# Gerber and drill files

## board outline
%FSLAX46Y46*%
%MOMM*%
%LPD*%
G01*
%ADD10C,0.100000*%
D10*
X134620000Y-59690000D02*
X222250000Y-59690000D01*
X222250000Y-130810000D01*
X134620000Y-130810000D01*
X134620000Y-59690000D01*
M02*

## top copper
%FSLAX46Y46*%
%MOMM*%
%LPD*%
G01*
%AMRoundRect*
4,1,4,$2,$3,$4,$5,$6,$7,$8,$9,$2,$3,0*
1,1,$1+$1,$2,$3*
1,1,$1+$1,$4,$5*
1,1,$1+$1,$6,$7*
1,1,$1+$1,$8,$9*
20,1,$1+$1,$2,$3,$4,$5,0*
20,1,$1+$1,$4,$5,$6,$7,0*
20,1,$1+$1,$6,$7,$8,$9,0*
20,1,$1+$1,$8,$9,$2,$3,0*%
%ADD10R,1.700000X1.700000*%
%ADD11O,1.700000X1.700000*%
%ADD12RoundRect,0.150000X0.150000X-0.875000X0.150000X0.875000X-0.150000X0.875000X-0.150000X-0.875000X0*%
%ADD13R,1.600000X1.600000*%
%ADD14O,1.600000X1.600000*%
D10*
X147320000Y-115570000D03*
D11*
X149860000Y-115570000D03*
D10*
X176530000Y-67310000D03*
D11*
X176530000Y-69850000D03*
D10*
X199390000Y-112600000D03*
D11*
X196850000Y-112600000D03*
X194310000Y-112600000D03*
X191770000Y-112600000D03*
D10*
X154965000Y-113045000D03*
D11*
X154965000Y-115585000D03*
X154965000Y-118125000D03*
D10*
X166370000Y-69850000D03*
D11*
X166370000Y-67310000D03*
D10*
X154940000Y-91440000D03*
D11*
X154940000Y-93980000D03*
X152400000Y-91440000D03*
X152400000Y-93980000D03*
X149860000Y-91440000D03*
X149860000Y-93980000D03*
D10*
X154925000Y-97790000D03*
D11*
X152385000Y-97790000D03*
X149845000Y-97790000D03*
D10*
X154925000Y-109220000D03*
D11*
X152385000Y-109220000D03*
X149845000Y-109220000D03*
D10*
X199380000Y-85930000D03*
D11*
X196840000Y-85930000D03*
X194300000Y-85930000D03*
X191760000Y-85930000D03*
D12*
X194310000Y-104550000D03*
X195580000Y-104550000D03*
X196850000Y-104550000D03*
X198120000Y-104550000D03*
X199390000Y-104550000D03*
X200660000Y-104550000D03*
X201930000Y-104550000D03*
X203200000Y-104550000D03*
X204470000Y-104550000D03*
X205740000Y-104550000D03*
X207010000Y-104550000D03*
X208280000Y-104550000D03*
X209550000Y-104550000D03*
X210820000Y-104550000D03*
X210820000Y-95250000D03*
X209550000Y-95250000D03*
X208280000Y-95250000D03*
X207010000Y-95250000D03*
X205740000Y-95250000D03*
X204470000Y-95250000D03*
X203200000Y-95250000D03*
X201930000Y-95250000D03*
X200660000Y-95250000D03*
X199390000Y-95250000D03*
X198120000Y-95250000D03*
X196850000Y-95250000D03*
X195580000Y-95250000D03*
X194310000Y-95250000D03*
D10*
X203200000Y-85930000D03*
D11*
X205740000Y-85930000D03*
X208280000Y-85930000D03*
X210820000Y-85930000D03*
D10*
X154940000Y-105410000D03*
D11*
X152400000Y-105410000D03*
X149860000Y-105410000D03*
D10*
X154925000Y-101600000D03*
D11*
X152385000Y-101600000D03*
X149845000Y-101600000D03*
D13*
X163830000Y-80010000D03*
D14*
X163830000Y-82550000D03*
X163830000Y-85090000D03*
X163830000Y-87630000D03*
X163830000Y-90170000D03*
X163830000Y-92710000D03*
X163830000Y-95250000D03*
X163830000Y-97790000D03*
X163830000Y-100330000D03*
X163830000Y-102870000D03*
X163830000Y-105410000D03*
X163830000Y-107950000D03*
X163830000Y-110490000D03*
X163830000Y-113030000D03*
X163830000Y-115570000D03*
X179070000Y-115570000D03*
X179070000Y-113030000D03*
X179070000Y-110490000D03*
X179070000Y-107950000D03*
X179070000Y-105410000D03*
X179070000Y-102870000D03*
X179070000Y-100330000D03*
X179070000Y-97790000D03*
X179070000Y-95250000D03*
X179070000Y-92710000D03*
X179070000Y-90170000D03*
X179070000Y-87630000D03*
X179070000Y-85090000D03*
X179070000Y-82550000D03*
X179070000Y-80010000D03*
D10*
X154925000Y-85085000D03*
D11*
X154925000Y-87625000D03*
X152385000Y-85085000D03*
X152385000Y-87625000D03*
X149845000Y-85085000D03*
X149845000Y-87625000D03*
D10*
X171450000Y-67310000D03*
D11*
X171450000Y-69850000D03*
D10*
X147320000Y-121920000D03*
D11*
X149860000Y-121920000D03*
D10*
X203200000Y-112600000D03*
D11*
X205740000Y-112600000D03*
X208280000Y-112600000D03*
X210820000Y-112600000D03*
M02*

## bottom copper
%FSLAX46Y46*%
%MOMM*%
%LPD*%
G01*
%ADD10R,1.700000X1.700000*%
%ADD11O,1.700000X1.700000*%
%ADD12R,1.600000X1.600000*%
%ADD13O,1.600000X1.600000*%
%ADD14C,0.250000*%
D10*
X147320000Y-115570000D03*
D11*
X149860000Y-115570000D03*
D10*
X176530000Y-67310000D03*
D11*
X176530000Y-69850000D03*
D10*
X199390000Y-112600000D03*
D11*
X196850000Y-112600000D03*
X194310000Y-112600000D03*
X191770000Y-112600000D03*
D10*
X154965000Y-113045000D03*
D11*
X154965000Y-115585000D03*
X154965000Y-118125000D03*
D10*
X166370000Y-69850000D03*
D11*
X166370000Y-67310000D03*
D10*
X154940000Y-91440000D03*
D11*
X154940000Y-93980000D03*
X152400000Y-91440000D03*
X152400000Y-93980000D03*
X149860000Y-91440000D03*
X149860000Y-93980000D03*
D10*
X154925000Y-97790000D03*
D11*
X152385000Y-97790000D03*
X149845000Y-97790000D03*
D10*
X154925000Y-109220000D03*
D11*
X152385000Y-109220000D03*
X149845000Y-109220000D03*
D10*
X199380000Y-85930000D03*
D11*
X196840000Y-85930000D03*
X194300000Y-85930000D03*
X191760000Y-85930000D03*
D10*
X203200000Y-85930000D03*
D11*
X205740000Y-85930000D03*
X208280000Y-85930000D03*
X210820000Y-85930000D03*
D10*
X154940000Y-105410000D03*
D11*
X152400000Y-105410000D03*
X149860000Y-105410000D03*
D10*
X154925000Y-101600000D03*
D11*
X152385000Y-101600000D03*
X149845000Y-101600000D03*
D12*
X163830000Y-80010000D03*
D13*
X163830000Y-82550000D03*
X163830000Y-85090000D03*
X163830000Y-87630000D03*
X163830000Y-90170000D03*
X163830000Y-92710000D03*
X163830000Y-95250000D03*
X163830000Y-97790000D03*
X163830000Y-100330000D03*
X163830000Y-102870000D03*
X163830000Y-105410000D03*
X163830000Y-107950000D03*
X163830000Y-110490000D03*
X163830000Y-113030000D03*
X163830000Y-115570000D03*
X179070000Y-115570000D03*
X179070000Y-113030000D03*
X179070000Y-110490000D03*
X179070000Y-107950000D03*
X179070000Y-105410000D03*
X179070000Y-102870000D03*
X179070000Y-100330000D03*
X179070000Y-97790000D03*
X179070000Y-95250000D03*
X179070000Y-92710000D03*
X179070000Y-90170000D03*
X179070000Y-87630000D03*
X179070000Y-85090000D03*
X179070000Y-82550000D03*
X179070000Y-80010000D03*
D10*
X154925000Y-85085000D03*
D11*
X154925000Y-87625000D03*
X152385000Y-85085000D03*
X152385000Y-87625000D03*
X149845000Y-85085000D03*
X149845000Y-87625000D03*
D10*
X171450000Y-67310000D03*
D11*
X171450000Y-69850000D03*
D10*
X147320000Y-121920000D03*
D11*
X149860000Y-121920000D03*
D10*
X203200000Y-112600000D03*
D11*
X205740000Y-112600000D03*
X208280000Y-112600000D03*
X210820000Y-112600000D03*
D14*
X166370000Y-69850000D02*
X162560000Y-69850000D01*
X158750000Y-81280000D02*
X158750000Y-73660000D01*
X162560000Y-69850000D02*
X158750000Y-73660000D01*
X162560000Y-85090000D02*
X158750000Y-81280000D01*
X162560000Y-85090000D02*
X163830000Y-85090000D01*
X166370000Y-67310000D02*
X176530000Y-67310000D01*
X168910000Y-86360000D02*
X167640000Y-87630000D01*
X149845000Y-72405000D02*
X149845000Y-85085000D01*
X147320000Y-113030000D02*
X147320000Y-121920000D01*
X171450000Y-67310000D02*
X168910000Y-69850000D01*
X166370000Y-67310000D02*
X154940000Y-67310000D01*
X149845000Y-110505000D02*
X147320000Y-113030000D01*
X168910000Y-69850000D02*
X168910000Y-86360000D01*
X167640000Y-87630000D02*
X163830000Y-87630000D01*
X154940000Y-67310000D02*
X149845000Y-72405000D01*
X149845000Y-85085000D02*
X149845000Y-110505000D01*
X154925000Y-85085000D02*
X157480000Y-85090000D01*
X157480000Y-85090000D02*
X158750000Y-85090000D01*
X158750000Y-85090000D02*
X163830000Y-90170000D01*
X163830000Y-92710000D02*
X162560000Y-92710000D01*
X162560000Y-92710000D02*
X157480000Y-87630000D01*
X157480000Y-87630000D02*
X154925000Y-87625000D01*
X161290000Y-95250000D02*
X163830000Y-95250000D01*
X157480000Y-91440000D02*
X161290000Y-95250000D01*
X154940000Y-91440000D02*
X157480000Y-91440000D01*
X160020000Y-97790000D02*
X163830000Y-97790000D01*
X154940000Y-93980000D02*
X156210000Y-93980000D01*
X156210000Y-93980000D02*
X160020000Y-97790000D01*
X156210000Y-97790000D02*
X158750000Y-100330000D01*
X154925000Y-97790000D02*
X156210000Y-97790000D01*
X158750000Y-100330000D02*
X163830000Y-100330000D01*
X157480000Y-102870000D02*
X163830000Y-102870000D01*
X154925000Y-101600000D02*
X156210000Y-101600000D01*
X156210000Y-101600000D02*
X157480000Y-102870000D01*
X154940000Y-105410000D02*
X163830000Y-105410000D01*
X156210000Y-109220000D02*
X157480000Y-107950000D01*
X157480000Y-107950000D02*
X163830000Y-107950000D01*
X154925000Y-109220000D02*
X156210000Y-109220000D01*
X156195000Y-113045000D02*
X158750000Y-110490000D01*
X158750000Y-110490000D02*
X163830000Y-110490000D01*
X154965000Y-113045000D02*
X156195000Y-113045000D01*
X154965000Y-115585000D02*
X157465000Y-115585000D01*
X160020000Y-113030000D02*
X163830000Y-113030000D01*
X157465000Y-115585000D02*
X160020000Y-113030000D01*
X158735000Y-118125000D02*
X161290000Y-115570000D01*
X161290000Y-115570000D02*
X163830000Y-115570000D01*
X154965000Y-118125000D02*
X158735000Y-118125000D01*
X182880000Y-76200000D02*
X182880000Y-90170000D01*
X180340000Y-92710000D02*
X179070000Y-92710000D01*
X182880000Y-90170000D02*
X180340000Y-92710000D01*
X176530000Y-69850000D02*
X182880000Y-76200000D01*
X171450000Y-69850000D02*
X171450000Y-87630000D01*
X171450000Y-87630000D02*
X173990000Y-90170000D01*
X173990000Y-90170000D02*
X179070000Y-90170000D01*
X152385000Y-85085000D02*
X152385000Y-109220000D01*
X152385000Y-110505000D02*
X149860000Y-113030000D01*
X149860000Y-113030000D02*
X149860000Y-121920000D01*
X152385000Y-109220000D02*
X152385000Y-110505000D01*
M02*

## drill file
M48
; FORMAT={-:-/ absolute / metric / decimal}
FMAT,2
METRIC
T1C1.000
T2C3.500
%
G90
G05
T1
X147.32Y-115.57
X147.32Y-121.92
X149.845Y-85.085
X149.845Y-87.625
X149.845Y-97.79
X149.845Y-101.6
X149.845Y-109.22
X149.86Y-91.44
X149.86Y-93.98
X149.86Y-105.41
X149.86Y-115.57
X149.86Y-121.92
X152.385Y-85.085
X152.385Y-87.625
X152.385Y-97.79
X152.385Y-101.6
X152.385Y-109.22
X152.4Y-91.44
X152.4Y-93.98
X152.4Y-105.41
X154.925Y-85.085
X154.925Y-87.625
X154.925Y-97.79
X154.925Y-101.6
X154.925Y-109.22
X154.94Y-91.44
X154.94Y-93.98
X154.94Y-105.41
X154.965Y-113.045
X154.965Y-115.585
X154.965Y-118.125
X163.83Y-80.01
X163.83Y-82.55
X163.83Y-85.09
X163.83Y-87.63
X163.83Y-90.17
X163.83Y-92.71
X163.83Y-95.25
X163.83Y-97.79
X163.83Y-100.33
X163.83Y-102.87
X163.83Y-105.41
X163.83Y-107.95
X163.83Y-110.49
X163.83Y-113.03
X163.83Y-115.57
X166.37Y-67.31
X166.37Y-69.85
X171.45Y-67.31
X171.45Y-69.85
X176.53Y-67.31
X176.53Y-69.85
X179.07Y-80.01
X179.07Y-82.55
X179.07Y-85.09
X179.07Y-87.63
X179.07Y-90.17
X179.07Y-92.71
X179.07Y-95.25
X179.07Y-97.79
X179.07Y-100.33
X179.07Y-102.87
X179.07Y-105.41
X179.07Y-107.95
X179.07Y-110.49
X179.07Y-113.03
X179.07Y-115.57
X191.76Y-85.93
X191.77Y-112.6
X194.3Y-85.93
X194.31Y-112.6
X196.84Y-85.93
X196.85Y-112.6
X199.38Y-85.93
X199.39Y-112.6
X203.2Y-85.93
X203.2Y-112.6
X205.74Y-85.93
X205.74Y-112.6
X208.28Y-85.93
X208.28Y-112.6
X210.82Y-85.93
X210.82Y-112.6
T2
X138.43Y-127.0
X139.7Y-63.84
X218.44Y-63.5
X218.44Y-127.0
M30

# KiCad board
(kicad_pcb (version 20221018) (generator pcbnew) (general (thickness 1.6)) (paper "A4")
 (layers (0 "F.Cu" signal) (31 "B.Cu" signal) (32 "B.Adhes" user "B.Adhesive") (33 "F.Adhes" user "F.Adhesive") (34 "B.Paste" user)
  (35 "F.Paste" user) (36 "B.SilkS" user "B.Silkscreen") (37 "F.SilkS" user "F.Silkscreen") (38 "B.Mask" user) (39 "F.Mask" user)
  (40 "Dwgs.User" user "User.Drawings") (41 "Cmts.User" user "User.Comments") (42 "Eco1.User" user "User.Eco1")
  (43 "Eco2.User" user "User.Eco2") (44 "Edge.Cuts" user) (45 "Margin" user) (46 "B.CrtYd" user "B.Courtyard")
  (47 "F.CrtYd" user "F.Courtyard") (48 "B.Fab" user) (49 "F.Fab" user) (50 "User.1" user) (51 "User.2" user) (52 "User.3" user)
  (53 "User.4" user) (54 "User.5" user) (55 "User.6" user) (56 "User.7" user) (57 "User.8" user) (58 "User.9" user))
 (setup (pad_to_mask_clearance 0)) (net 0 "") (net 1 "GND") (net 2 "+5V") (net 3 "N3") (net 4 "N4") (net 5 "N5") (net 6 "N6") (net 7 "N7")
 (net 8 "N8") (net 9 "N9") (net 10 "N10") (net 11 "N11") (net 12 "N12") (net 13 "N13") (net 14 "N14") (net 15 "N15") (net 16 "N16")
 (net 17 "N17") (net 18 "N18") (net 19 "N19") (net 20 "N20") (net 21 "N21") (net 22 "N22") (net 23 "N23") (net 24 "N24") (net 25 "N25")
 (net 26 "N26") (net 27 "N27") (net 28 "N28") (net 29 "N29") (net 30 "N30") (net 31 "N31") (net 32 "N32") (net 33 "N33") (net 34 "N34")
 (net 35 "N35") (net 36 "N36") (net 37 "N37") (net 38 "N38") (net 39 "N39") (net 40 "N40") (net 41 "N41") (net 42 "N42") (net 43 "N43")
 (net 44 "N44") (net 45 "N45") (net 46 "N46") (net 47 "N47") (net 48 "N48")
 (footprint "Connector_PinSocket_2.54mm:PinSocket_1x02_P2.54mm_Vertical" (layer "F.Cu") (at 147.32 115.57 90)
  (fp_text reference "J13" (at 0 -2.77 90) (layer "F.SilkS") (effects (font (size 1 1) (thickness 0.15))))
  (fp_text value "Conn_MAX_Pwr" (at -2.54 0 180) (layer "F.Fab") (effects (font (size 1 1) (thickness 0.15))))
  (pad "1" thru_hole rect (at 0 0 90) (size 1.7 1.7) (drill 1) (layers "*.Cu" "*.Mask") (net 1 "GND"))
  (pad "2" thru_hole oval (at 0 2.54 90) (size 1.7 1.7) (drill 1) (layers "*.Cu" "*.Mask") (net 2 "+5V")))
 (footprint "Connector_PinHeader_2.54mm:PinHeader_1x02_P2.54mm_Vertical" (layer "F.Cu") (at 176.53 67.31)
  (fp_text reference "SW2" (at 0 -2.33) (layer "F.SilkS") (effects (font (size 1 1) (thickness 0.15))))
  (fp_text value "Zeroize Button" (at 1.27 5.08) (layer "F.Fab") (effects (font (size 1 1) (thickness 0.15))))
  (pad "1" thru_hole rect (at 0 0) (size 1.7 1.7) (drill 1) (layers "*.Cu" "*.Mask") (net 1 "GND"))
  (pad "2" thru_hole oval (at 0 2.54) (size 1.7 1.7) (drill 1) (layers "*.Cu" "*.Mask") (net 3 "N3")))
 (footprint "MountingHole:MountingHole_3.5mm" (layer "F.Cu") (at 139.7 63.84)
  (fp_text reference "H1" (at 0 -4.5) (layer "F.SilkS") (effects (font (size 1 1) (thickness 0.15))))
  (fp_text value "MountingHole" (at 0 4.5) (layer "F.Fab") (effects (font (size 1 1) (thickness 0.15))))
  (pad "" np_thru_hole circle (at 0 0) (size 3.5 3.5) (drill 3.5) (layers "*.Cu" "*.Mask")))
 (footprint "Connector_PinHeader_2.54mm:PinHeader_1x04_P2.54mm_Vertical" (layer "F.Cu") (at 199.39 112.6 -90)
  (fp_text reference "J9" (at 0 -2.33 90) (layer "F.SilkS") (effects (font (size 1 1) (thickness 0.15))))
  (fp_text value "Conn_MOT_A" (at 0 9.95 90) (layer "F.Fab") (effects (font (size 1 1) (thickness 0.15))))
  (pad "1" thru_hole rect (at 0 0 270) (size 1.7 1.7) (drill 1) (layers "*.Cu" "*.Mask") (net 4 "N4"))
  (pad "2" thru_hole oval (at 0 2.54 270) (size 1.7 1.7) (drill 1) (layers "*.Cu" "*.Mask") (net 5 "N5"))
  (pad "3" thru_hole oval (at 0 5.08 270) (size 1.7 1.7) (drill 1) (layers "*.Cu" "*.Mask") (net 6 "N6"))
  (pad "4" thru_hole oval (at 0 7.62 270) (size 1.7 1.7) (drill 1) (layers "*.Cu" "*.Mask") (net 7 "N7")))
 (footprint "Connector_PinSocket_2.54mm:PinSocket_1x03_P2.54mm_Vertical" (layer "F.Cu") (at 154.965 113.045)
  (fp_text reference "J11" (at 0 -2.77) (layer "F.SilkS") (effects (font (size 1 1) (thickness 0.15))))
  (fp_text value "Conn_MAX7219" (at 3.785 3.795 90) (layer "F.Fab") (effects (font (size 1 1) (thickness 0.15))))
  (pad "1" thru_hole rect (at 0 0) (size 1.7 1.7) (drill 1) (layers "*.Cu" "*.Mask") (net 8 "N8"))
  (pad "2" thru_hole oval (at 0 2.54) (size 1.7 1.7) (drill 1) (layers "*.Cu" "*.Mask") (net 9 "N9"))
  (pad "3" thru_hole oval (at 0 5.08) (size 1.7 1.7) (drill 1) (layers "*.Cu" "*.Mask") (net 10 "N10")))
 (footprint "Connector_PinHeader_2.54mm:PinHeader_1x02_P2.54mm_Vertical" (layer "F.Cu") (at 166.37 69.85 180)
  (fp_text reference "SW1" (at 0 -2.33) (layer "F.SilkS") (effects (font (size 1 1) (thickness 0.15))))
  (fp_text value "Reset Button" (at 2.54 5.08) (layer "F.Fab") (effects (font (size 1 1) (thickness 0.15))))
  (pad "1" thru_hole rect (at 0 0 180) (size 1.7 1.7) (drill 1) (layers "*.Cu" "*.Mask") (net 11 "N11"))
  (pad "2" thru_hole oval (at 0 2.54 180) (size 1.7 1.7) (drill 1) (layers "*.Cu" "*.Mask") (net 1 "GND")))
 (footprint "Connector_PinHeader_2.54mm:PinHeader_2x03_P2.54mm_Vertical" (layer "F.Cu") (at 154.94 91.44 -90)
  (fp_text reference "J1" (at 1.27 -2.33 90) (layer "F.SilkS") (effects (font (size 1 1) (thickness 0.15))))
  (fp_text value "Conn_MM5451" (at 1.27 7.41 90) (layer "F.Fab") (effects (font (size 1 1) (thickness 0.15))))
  (pad "1" thru_hole rect (at 0 0 270) (size 1.7 1.7) (drill 1) (layers "*.Cu" "*.Mask") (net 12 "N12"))
  (pad "2" thru_hole oval (at 2.54 0 270) (size 1.7 1.7) (drill 1) (layers "*.Cu" "*.Mask") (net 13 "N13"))
  (pad "3" thru_hole oval (at 0 2.54 270) (size 1.7 1.7) (drill 1) (layers "*.Cu" "*.Mask") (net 2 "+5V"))
  (pad "4" thru_hole oval (at 2.54 2.54 270) (size 1.7 1.7) (drill 1) (layers "*.Cu" "*.Mask") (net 2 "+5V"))
  (pad "5" thru_hole oval (at 0 5.08 270) (size 1.7 1.7) (drill 1) (layers "*.Cu" "*.Mask") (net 1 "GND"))
  (pad "6" thru_hole oval (at 2.54 5.08 270) (size 1.7 1.7) (drill 1) (layers "*.Cu" "*.Mask") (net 1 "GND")))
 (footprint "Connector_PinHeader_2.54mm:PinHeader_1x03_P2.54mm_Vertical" (layer "F.Cu") (at 154.925 97.79 -90)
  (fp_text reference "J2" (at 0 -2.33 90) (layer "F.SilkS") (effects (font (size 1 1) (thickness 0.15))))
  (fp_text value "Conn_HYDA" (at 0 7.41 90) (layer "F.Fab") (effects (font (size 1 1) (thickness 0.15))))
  (pad "1" thru_hole rect (at 0 0 270) (size 1.7 1.7) (drill 1) (layers "*.Cu" "*.Mask") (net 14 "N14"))
  (pad "2" thru_hole oval (at 0 2.54 270) (size 1.7 1.7) (drill 1) (layers "*.Cu" "*.Mask") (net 2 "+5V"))
  (pad "3" thru_hole oval (at 0 5.08 270) (size 1.7 1.7) (drill 1) (layers "*.Cu" "*.Mask") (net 1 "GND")))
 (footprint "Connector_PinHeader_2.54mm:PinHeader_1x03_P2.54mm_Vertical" (layer "F.Cu") (at 154.925 109.22 -90)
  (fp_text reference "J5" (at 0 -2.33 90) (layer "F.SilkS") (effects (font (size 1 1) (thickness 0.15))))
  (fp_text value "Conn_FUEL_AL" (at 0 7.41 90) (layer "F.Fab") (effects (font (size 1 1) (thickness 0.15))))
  (pad "1" thru_hole rect (at 0 0 270) (size 1.7 1.7) (drill 1) (layers "*.Cu" "*.Mask") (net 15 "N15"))
  (pad "2" thru_hole oval (at 0 2.54 270) (size 1.7 1.7) (drill 1) (layers "*.Cu" "*.Mask") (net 2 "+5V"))
  (pad "3" thru_hole oval (at 0 5.08 270) (size 1.7 1.7) (drill 1) (layers "*.Cu" "*.Mask") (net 1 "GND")))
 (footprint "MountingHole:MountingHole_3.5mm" (layer "F.Cu") (at 218.44 127)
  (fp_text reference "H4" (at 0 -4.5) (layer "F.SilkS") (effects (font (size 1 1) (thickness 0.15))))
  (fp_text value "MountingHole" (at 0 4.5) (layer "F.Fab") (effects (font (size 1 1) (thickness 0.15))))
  (pad "" np_thru_hole circle (at 0 0) (size 3.5 3.5) (drill 3.5) (layers "*.Cu" "*.Mask")))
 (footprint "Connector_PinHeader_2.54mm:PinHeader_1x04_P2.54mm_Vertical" (layer "F.Cu") (at 199.38 85.93 -90)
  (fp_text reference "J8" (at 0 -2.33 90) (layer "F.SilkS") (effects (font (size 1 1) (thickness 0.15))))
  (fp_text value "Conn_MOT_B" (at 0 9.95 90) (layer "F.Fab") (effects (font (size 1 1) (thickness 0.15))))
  (pad "1" thru_hole rect (at 0 0 270) (size 1.7 1.7) (drill 1) (layers "*.Cu" "*.Mask") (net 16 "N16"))
  (pad "2" thru_hole oval (at 0 2.54 270) (size 1.7 1.7) (drill 1) (layers "*.Cu" "*.Mask") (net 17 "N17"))
  (pad "3" thru_hole oval (at 0 5.08 270) (size 1.7 1.7) (drill 1) (layers "*.Cu" "*.Mask") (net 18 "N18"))
  (pad "4" thru_hole oval (at 0 7.62 270) (size 1.7 1.7) (drill 1) (layers "*.Cu" "*.Mask") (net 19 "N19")))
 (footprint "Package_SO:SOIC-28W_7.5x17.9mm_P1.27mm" (layer "F.Cu") (at 202.565 99.9 90)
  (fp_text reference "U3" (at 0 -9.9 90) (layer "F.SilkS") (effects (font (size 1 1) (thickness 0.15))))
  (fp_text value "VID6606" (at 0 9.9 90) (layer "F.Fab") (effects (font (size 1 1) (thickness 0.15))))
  (pad "1" smd roundrect (at -4.65 -8.255 90) (size 2.05 0.6) (layers "F.Cu" "F.Paste" "F.Mask") (roundrect_rratio 0.25) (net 1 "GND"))
  (pad "2" smd roundrect (at -4.65 -6.985 90) (size 2.05 0.6) (layers "F.Cu" "F.Paste" "F.Mask") (roundrect_rratio 0.25) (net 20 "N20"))
  (pad "3" smd roundrect (at -4.65 -5.715 90) (size 2.05 0.6) (layers "F.Cu" "F.Paste" "F.Mask") (roundrect_rratio 0.25) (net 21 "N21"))
  (pad "4" smd roundrect (at -4.65 -4.445 90) (size 2.05 0.6) (layers "F.Cu" "F.Paste" "F.Mask") (roundrect_rratio 0.25) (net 7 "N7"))
  (pad "5" smd roundrect (at -4.65 -3.175 90) (size 2.05 0.6) (layers "F.Cu" "F.Paste" "F.Mask") (roundrect_rratio 0.25) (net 6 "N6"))
  (pad "6" smd roundrect (at -4.65 -1.905 90) (size 2.05 0.6) (layers "F.Cu" "F.Paste" "F.Mask") (roundrect_rratio 0.25) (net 5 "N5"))
  (pad "7" smd roundrect (at -4.65 -0.635 90) (size 2.05 0.6) (layers "F.Cu" "F.Paste" "F.Mask") (roundrect_rratio 0.25) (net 4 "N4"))
  (pad "8" smd roundrect (at -4.65 0.635 90) (size 2.05 0.6) (layers "F.Cu" "F.Paste" "F.Mask") (roundrect_rratio 0.25) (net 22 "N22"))
  (pad "9" smd roundrect (at -4.65 1.905 90) (size 2.05 0.6) (layers "F.Cu" "F.Paste" "F.Mask") (roundrect_rratio 0.25) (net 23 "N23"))
  (pad "10" smd roundrect (at -4.65 3.175 90) (size 2.05 0.6) (layers "F.Cu" "F.Paste" "F.Mask") (roundrect_rratio 0.25) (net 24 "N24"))
  (pad "11" smd roundrect (at -4.65 4.445 90) (size 2.05 0.6) (layers "F.Cu" "F.Paste" "F.Mask") (roundrect_rratio 0.25) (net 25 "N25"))
  (pad "12" smd roundrect (at -4.65 5.715 90) (size 2.05 0.6) (layers "F.Cu" "F.Paste" "F.Mask") (roundrect_rratio 0.25) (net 2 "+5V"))
  (pad "13" smd roundrect (at -4.65 6.985 90) (size 2.05 0.6) (layers "F.Cu" "F.Paste" "F.Mask") (roundrect_rratio 0.25) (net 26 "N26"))
  (pad "14" smd roundrect (at -4.65 8.255 90) (size 2.05 0.6) (layers "F.Cu" "F.Paste" "F.Mask") (roundrect_rratio 0.25) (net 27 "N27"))
  (pad "15" smd roundrect (at 4.65 8.255 90) (size 2.05 0.6) (layers "F.Cu" "F.Paste" "F.Mask") (roundrect_rratio 0.25) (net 1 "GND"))
  (pad "16" smd roundrect (at 4.65 6.985 90) (size 2.05 0.6) (layers "F.Cu" "F.Paste" "F.Mask") (roundrect_rratio 0.25) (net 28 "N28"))
  (pad "17" smd roundrect (at 4.65 5.715 90) (size 2.05 0.6) (layers "F.Cu" "F.Paste" "F.Mask") (roundrect_rratio 0.25) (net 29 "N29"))
  (pad "18" smd roundrect (at 4.65 4.445 90) (size 2.05 0.6) (layers "F.Cu" "F.Paste" "F.Mask") (roundrect_rratio 0.25) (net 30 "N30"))
  (pad "19" smd roundrect (at 4.65 3.175 90) (size 2.05 0.6) (layers "F.Cu" "F.Paste" "F.Mask") (roundrect_rratio 0.25) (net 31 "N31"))
  (pad "20" smd roundrect (at 4.65 1.905 90) (size 2.05 0.6) (layers "F.Cu" "F.Paste" "F.Mask") (roundrect_rratio 0.25) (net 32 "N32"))
  (pad "21" smd roundrect (at 4.65 0.635 90) (size 2.05 0.6) (layers "F.Cu" "F.Paste" "F.Mask") (roundrect_rratio 0.25) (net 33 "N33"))
  (pad "22" smd roundrect (at 4.65 -0.635 90) (size 2.05 0.6) (layers "F.Cu" "F.Paste" "F.Mask") (roundrect_rratio 0.25) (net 16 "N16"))
  (pad "23" smd roundrect (at 4.65 -1.905 90) (size 2.05 0.6) (layers "F.Cu" "F.Paste" "F.Mask") (roundrect_rratio 0.25) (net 17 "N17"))
  (pad "24" smd roundrect (at 4.65 -3.175 90) (size 2.05 0.6) (layers "F.Cu" "F.Paste" "F.Mask") (roundrect_rratio 0.25) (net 18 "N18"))
  (pad "25" smd roundrect (at 4.65 -4.445 90) (size 2.05 0.6) (layers "F.Cu" "F.Paste" "F.Mask") (roundrect_rratio 0.25) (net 19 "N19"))
  (pad "26" smd roundrect (at 4.65 -5.715 90) (size 2.05 0.6) (layers "F.Cu" "F.Paste" "F.Mask") (roundrect_rratio 0.25) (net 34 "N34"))
  (pad "27" smd roundrect (at 4.65 -6.985 90) (size 2.05 0.6) (layers "F.Cu" "F.Paste" "F.Mask") (roundrect_rratio 0.25) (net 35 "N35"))
  (pad "28" smd roundrect (at 4.65 -8.255 90) (size 2.05 0.6) (layers "F.Cu" "F.Paste" "F.Mask") (roundrect_rratio 0.25) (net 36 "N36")))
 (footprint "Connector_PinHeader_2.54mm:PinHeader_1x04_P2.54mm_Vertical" (layer "F.Cu") (at 203.2 85.93 90)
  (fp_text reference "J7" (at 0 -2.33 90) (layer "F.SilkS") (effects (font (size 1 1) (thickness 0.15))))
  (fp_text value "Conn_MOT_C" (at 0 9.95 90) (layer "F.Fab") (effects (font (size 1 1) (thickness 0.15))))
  (pad "1" thru_hole rect (at 0 0 90) (size 1.7 1.7) (drill 1) (layers "*.Cu" "*.Mask") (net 33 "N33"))
  (pad "2" thru_hole oval (at 0 2.54 90) (size 1.7 1.7) (drill 1) (layers "*.Cu" "*.Mask") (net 32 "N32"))
  (pad "3" thru_hole oval (at 0 5.08 90) (size 1.7 1.7) (drill 1) (layers "*.Cu" "*.Mask") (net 31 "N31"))
  (pad "4" thru_hole oval (at 0 7.62 90) (size 1.7 1.7) (drill 1) (layers "*.Cu" "*.Mask") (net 30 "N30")))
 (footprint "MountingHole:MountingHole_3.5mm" (layer "F.Cu") (at 218.44 63.5)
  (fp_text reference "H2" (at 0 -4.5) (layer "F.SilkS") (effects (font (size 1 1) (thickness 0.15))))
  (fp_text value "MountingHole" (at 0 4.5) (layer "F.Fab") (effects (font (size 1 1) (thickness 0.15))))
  (pad "" np_thru_hole circle (at 0 0) (size 3.5 3.5) (drill 3.5) (layers "*.Cu" "*.Mask")))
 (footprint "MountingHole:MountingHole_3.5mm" (layer "F.Cu") (at 138.43 127)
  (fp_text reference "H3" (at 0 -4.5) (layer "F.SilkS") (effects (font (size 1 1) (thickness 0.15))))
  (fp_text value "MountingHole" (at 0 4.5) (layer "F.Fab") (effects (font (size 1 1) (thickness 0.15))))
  (pad "" np_thru_hole circle (at 0 0) (size 3.5 3.5) (drill 3.5) (layers "*.Cu" "*.Mask")))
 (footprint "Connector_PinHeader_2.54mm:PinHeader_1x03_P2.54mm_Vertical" (layer "F.Cu") (at 154.94 105.41 -90)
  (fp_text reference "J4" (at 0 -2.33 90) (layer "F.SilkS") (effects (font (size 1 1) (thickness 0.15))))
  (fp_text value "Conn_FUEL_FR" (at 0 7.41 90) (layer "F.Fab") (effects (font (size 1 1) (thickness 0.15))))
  (pad "1" thru_hole rect (at 0 0 270) (size 1.7 1.7) (drill 1) (layers "*.Cu" "*.Mask") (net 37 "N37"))
  (pad "2" thru_hole oval (at 0 2.54 270) (size 1.7 1.7) (drill 1) (layers "*.Cu" "*.Mask") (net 2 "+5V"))
  (pad "3" thru_hole oval (at 0 5.08 270) (size 1.7 1.7) (drill 1) (layers "*.Cu" "*.Mask") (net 1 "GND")))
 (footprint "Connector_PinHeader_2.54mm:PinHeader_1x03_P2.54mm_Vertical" (layer "F.Cu") (at 154.925 101.6 -90)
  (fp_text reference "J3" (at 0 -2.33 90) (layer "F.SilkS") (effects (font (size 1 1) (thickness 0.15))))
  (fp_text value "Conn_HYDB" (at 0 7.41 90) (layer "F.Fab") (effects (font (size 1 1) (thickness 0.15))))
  (pad "1" thru_hole rect (at 0 0 270) (size 1.7 1.7) (drill 1) (layers "*.Cu" "*.Mask") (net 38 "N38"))
  (pad "2" thru_hole oval (at 0 2.54 270) (size 1.7 1.7) (drill 1) (layers "*.Cu" "*.Mask") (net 2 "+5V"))
  (pad "3" thru_hole oval (at 0 5.08 270) (size 1.7 1.7) (drill 1) (layers "*.Cu" "*.Mask") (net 1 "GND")))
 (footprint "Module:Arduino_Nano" (layer "F.Cu") (at 163.83 80.01)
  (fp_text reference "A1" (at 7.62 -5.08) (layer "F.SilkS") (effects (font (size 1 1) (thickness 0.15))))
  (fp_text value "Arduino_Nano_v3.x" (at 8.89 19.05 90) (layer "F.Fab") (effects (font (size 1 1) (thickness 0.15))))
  (pad "1" thru_hole rect (at 0 0) (size 1.6 1.6) (drill 1) (layers "*.Cu" "*.Mask") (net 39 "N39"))
  (pad "2" thru_hole oval (at 0 2.54) (size 1.6 1.6) (drill 1) (layers "*.Cu" "*.Mask") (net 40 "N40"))
  (pad "3" thru_hole oval (at 0 5.08) (size 1.6 1.6) (drill 1) (layers "*.Cu" "*.Mask") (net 11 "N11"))
  (pad "4" thru_hole oval (at 0 7.62) (size 1.6 1.6) (drill 1) (layers "*.Cu" "*.Mask") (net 1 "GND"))
  (pad "5" thru_hole oval (at 0 10.16) (size 1.6 1.6) (drill 1) (layers "*.Cu" "*.Mask") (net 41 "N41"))
  (pad "6" thru_hole oval (at 0 12.7) (size 1.6 1.6) (drill 1) (layers "*.Cu" "*.Mask") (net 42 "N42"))
  (pad "7" thru_hole oval (at 0 15.24) (size 1.6 1.6) (drill 1) (layers "*.Cu" "*.Mask") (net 12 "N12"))
  (pad "8" thru_hole oval (at 0 17.78) (size 1.6 1.6) (drill 1) (layers "*.Cu" "*.Mask") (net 13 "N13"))
  (pad "9" thru_hole oval (at 0 20.32) (size 1.6 1.6) (drill 1) (layers "*.Cu" "*.Mask") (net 14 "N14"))
  (pad "10" thru_hole oval (at 0 22.86) (size 1.6 1.6) (drill 1) (layers "*.Cu" "*.Mask") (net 38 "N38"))
  (pad "11" thru_hole oval (at 0 25.4) (size 1.6 1.6) (drill 1) (layers "*.Cu" "*.Mask") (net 37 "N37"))
  (pad "12" thru_hole oval (at 0 27.94) (size 1.6 1.6) (drill 1) (layers "*.Cu" "*.Mask") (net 15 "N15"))
  (pad "13" thru_hole oval (at 0 30.48) (size 1.6 1.6) (drill 1) (layers "*.Cu" "*.Mask") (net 8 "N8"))
  (pad "14" thru_hole oval (at 0 33.02) (size 1.6 1.6) (drill 1) (layers "*.Cu" "*.Mask") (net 9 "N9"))
  (pad "15" thru_hole oval (at 0 35.56) (size 1.6 1.6) (drill 1) (layers "*.Cu" "*.Mask") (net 10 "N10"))
  (pad "16" thru_hole oval (at 15.24 35.56) (size 1.6 1.6) (drill 1) (layers "*.Cu" "*.Mask") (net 34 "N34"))
  (pad "17" thru_hole oval (at 15.24 33.02) (size 1.6 1.6) (drill 1) (layers "*.Cu" "*.Mask") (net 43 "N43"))
  (pad "18" thru_hole oval (at 15.24 30.48) (size 1.6 1.6) (drill 1) (layers "*.Cu" "*.Mask") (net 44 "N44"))
  (pad "19" thru_hole oval (at 15.24 27.94) (size 1.6 1.6) (drill 1) (layers "*.Cu" "*.Mask") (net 26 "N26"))
  (pad "20" thru_hole oval (at 15.24 25.4) (size 1.6 1.6) (drill 1) (layers "*.Cu" "*.Mask") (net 27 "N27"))
  (pad "21" thru_hole oval (at 15.24 22.86) (size 1.6 1.6) (drill 1) (layers "*.Cu" "*.Mask") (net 20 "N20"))
  (pad "22" thru_hole oval (at 15.24 20.32) (size 1.6 1.6) (drill 1) (layers "*.Cu" "*.Mask") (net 21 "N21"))
  (pad "23" thru_hole oval (at 15.24 17.78) (size 1.6 1.6) (drill 1) (layers "*.Cu" "*.Mask") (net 35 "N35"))
  (pad "24" thru_hole oval (at 15.24 15.24) (size 1.6 1.6) (drill 1) (layers "*.Cu" "*.Mask") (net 36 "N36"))
  (pad "25" thru_hole oval (at 15.24 12.7) (size 1.6 1.6) (drill 1) (layers "*.Cu" "*.Mask") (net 3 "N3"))
  (pad "26" thru_hole oval (at 15.24 10.16) (size 1.6 1.6) (drill 1) (layers "*.Cu" "*.Mask") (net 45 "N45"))
  (pad "27" thru_hole oval (at 15.24 7.62) (size 1.6 1.6) (drill 1) (layers "*.Cu" "*.Mask") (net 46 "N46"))
  (pad "28" thru_hole oval (at 15.24 5.08) (size 1.6 1.6) (drill 1) (layers "*.Cu" "*.Mask") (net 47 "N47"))
  (pad "29" thru_hole oval (at 15.24 2.54) (size 1.6 1.6) (drill 1) (layers "*.Cu" "*.Mask") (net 1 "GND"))
  (pad "30" thru_hole oval (at 15.24 0) (size 1.6 1.6) (drill 1) (layers "*.Cu" "*.Mask") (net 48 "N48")))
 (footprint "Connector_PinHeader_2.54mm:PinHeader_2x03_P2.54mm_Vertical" (layer "F.Cu") (at 154.925 85.085 -90)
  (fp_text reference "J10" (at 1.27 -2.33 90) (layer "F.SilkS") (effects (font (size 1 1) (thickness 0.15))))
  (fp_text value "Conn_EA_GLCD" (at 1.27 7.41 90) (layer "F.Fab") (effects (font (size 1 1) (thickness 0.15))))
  (pad "1" thru_hole rect (at 0 0 270) (size 1.7 1.7) (drill 1) (layers "*.Cu" "*.Mask") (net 41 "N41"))
  (pad "2" thru_hole oval (at 2.54 0 270) (size 1.7 1.7) (drill 1) (layers "*.Cu" "*.Mask") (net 42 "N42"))
  (pad "3" thru_hole oval (at 0 2.54 270) (size 1.7 1.7) (drill 1) (layers "*.Cu" "*.Mask") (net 2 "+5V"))
  (pad "4" thru_hole oval (at 2.54 2.54 270) (size 1.7 1.7) (drill 1) (layers "*.Cu" "*.Mask") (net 2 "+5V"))
  (pad "5" thru_hole oval (at 0 5.08 270) (size 1.7 1.7) (drill 1) (layers "*.Cu" "*.Mask") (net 1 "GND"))
  (pad "6" thru_hole oval (at 2.54 5.08 270) (size 1.7 1.7) (drill 1) (layers "*.Cu" "*.Mask") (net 1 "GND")))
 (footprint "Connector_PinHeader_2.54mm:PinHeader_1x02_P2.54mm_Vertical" (layer "F.Cu") (at 171.45 67.31)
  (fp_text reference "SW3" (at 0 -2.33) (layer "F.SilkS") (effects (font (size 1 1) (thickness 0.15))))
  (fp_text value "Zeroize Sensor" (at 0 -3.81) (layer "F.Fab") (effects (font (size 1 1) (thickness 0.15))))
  (pad "1" thru_hole rect (at 0 0) (size 1.7 1.7) (drill 1) (layers "*.Cu" "*.Mask") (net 1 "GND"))
  (pad "2" thru_hole oval (at 0 2.54) (size 1.7 1.7) (drill 1) (layers "*.Cu" "*.Mask") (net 45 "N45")))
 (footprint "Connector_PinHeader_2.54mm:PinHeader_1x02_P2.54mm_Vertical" (layer "F.Cu") (at 147.32 121.92 90)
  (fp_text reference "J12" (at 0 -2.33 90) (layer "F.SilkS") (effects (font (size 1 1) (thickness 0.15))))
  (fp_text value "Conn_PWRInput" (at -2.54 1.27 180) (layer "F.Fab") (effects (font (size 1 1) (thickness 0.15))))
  (pad "1" thru_hole rect (at 0 0 90) (size 1.7 1.7) (drill 1) (layers "*.Cu" "*.Mask") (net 1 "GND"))
  (pad "2" thru_hole oval (at 0 2.54 90) (size 1.7 1.7) (drill 1) (layers "*.Cu" "*.Mask") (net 2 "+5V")))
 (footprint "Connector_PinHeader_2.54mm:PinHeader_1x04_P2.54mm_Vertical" (layer "F.Cu") (at 203.2 112.6 90)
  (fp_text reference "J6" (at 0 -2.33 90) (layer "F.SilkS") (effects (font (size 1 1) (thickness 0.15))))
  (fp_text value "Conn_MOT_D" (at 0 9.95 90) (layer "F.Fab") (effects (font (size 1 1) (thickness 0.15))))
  (pad "1" thru_hole rect (at 0 0 90) (size 1.7 1.7) (drill 1) (layers "*.Cu" "*.Mask") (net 22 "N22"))
  (pad "2" thru_hole oval (at 0 2.54 90) (size 1.7 1.7) (drill 1) (layers "*.Cu" "*.Mask") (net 23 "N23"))
  (pad "3" thru_hole oval (at 0 5.08 90) (size 1.7 1.7) (drill 1) (layers "*.Cu" "*.Mask") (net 24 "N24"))
  (pad "4" thru_hole oval (at 0 7.62 90) (size 1.7 1.7) (drill 1) (layers "*.Cu" "*.Mask") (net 25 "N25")))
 (gr_rect (start 134.62 59.69) (end 222.25 130.81) (stroke (width 0.1) (type default)) (fill none) (layer "Edge.Cuts"))
 (segment (start 166.37 69.85) (end 162.56 69.85) (width 0.25) (layer "B.Cu") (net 11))
 (segment (start 158.75 81.28) (end 158.75 73.66) (width 0.25) (layer "B.Cu") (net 11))
 (segment (start 162.56 69.85) (end 158.75 73.66) (width 0.25) (layer "B.Cu") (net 11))
 (segment (start 162.56 85.09) (end 158.75 81.28) (width 0.25) (layer "B.Cu") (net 11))
 (segment (start 162.56 85.09) (end 163.83 85.09) (width 0.25) (layer "B.Cu") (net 11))
 (segment (start 166.37 67.31) (end 176.53 67.31) (width 0.25) (layer "B.Cu") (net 1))
 (segment (start 168.91 86.36) (end 167.64 87.63) (width 0.25) (layer "B.Cu") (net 1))
 (segment (start 149.845 72.405) (end 149.845 85.085) (width 0.25) (layer "B.Cu") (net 1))
 (segment (start 147.32 113.03) (end 147.32 121.92) (width 0.25) (layer "B.Cu") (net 1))
 (segment (start 171.45 67.31) (end 168.91 69.85) (width 0.25) (layer "B.Cu") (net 1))
 (segment (start 166.37 67.31) (end 154.94 67.31) (width 0.25) (layer "B.Cu") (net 1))
 (segment (start 149.845 110.505) (end 147.32 113.03) (width 0.25) (layer "B.Cu") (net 1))
 (segment (start 168.91 69.85) (end 168.91 86.36) (width 0.25) (layer "B.Cu") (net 1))
 (segment (start 167.64 87.63) (end 163.83 87.63) (width 0.25) (layer "B.Cu") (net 1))
 (segment (start 154.94 67.31) (end 149.845 72.405) (width 0.25) (layer "B.Cu") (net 1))
 (segment (start 149.845 85.085) (end 149.845 110.505) (width 0.25) (layer "B.Cu") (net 1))
 (segment (start 154.925 85.085) (end 157.48 85.09) (width 0.25) (layer "B.Cu") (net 41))
 (segment (start 157.48 85.09) (end 158.75 85.09) (width 0.25) (layer "B.Cu") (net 41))
 (segment (start 158.75 85.09) (end 163.83 90.17) (width 0.25) (layer "B.Cu") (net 41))
 (segment (start 163.83 92.71) (end 162.56 92.71) (width 0.25) (layer "B.Cu") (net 42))
 (segment (start 162.56 92.71) (end 157.48 87.63) (width 0.25) (layer "B.Cu") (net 42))
 (segment (start 157.48 87.63) (end 154.925 87.625) (width 0.25) (layer "B.Cu") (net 42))
 (segment (start 161.29 95.25) (end 163.83 95.25) (width 0.25) (layer "B.Cu") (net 12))
 (segment (start 157.48 91.44) (end 161.29 95.25) (width 0.25) (layer "B.Cu") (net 12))
 (segment (start 154.94 91.44) (end 157.48 91.44) (width 0.25) (layer "B.Cu") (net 12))
 (segment (start 160.02 97.79) (end 163.83 97.79) (width 0.25) (layer "B.Cu") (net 13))
 (segment (start 154.94 93.98) (end 156.21 93.98) (width 0.25) (layer "B.Cu") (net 13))
 (segment (start 156.21 93.98) (end 160.02 97.79) (width 0.25) (layer "B.Cu") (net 13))
 (segment (start 156.21 97.79) (end 158.75 100.33) (width 0.25) (layer "B.Cu") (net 14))
 (segment (start 154.925 97.79) (end 156.21 97.79) (width 0.25) (layer "B.Cu") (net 14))
 (segment (start 158.75 100.33) (end 163.83 100.33) (width 0.25) (layer "B.Cu") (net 14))
 (segment (start 157.48 102.87) (end 163.83 102.87) (width 0.25) (layer "B.Cu") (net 38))
 (segment (start 154.925 101.6) (end 156.21 101.6) (width 0.25) (layer "B.Cu") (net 38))
 (segment (start 156.21 101.6) (end 157.48 102.87) (width 0.25) (layer "B.Cu") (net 38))
 (segment (start 154.94 105.41) (end 163.83 105.41) (width 0.25) (layer "B.Cu") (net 37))
 (segment (start 156.21 109.22) (end 157.48 107.95) (width 0.25) (layer "B.Cu") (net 15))
 (segment (start 157.48 107.95) (end 163.83 107.95) (width 0.25) (layer "B.Cu") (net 15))
 (segment (start 154.925 109.22) (end 156.21 109.22) (width 0.25) (layer "B.Cu") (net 15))
 (segment (start 156.195 113.045) (end 158.75 110.49) (width 0.25) (layer "B.Cu") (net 8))
 (segment (start 158.75 110.49) (end 163.83 110.49) (width 0.25) (layer "B.Cu") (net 8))
 (segment (start 154.965 113.045) (end 156.195 113.045) (width 0.25) (layer "B.Cu") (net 8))
 (segment (start 154.965 115.585) (end 157.465 115.585) (width 0.25) (layer "B.Cu") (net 9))
 (segment (start 160.02 113.03) (end 163.83 113.03) (width 0.25) (layer "B.Cu") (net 9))
 (segment (start 157.465 115.585) (end 160.02 113.03) (width 0.25) (layer "B.Cu") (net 9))
 (segment (start 158.735 118.125) (end 161.29 115.57) (width 0.25) (layer "B.Cu") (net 10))
 (segment (start 161.29 115.57) (end 163.83 115.57) (width 0.25) (layer "B.Cu") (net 10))
 (segment (start 154.965 118.125) (end 158.735 118.125) (width 0.25) (layer "B.Cu") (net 10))
 (segment (start 182.88 76.2) (end 182.88 90.17) (width 0.25) (layer "B.Cu") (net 3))
 (segment (start 180.34 92.71) (end 179.07 92.71) (width 0.25) (layer "B.Cu") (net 3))
 (segment (start 182.88 90.17) (end 180.34 92.71) (width 0.25) (layer "B.Cu") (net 3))
 (segment (start 176.53 69.85) (end 182.88 76.2) (width 0.25) (layer "B.Cu") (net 3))
 (segment (start 171.45 69.85) (end 171.45 87.63) (width 0.25) (layer "B.Cu") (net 45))
 (segment (start 171.45 87.63) (end 173.99 90.17) (width 0.25) (layer "B.Cu") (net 45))
 (segment (start 173.99 90.17) (end 179.07 90.17) (width 0.25) (layer "B.Cu") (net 45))
 (segment (start 152.385 85.085) (end 152.385 109.22) (width 0.25) (layer "B.Cu") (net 2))
 (segment (start 152.385 110.505) (end 149.86 113.03) (width 0.25) (layer "B.Cu") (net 2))
 (segment (start 149.86 113.03) (end 149.86 121.92) (width 0.25) (layer "B.Cu") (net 2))
 (segment (start 152.385 109.22) (end 152.385 110.505) (width 0.25) (layer "B.Cu") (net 2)))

